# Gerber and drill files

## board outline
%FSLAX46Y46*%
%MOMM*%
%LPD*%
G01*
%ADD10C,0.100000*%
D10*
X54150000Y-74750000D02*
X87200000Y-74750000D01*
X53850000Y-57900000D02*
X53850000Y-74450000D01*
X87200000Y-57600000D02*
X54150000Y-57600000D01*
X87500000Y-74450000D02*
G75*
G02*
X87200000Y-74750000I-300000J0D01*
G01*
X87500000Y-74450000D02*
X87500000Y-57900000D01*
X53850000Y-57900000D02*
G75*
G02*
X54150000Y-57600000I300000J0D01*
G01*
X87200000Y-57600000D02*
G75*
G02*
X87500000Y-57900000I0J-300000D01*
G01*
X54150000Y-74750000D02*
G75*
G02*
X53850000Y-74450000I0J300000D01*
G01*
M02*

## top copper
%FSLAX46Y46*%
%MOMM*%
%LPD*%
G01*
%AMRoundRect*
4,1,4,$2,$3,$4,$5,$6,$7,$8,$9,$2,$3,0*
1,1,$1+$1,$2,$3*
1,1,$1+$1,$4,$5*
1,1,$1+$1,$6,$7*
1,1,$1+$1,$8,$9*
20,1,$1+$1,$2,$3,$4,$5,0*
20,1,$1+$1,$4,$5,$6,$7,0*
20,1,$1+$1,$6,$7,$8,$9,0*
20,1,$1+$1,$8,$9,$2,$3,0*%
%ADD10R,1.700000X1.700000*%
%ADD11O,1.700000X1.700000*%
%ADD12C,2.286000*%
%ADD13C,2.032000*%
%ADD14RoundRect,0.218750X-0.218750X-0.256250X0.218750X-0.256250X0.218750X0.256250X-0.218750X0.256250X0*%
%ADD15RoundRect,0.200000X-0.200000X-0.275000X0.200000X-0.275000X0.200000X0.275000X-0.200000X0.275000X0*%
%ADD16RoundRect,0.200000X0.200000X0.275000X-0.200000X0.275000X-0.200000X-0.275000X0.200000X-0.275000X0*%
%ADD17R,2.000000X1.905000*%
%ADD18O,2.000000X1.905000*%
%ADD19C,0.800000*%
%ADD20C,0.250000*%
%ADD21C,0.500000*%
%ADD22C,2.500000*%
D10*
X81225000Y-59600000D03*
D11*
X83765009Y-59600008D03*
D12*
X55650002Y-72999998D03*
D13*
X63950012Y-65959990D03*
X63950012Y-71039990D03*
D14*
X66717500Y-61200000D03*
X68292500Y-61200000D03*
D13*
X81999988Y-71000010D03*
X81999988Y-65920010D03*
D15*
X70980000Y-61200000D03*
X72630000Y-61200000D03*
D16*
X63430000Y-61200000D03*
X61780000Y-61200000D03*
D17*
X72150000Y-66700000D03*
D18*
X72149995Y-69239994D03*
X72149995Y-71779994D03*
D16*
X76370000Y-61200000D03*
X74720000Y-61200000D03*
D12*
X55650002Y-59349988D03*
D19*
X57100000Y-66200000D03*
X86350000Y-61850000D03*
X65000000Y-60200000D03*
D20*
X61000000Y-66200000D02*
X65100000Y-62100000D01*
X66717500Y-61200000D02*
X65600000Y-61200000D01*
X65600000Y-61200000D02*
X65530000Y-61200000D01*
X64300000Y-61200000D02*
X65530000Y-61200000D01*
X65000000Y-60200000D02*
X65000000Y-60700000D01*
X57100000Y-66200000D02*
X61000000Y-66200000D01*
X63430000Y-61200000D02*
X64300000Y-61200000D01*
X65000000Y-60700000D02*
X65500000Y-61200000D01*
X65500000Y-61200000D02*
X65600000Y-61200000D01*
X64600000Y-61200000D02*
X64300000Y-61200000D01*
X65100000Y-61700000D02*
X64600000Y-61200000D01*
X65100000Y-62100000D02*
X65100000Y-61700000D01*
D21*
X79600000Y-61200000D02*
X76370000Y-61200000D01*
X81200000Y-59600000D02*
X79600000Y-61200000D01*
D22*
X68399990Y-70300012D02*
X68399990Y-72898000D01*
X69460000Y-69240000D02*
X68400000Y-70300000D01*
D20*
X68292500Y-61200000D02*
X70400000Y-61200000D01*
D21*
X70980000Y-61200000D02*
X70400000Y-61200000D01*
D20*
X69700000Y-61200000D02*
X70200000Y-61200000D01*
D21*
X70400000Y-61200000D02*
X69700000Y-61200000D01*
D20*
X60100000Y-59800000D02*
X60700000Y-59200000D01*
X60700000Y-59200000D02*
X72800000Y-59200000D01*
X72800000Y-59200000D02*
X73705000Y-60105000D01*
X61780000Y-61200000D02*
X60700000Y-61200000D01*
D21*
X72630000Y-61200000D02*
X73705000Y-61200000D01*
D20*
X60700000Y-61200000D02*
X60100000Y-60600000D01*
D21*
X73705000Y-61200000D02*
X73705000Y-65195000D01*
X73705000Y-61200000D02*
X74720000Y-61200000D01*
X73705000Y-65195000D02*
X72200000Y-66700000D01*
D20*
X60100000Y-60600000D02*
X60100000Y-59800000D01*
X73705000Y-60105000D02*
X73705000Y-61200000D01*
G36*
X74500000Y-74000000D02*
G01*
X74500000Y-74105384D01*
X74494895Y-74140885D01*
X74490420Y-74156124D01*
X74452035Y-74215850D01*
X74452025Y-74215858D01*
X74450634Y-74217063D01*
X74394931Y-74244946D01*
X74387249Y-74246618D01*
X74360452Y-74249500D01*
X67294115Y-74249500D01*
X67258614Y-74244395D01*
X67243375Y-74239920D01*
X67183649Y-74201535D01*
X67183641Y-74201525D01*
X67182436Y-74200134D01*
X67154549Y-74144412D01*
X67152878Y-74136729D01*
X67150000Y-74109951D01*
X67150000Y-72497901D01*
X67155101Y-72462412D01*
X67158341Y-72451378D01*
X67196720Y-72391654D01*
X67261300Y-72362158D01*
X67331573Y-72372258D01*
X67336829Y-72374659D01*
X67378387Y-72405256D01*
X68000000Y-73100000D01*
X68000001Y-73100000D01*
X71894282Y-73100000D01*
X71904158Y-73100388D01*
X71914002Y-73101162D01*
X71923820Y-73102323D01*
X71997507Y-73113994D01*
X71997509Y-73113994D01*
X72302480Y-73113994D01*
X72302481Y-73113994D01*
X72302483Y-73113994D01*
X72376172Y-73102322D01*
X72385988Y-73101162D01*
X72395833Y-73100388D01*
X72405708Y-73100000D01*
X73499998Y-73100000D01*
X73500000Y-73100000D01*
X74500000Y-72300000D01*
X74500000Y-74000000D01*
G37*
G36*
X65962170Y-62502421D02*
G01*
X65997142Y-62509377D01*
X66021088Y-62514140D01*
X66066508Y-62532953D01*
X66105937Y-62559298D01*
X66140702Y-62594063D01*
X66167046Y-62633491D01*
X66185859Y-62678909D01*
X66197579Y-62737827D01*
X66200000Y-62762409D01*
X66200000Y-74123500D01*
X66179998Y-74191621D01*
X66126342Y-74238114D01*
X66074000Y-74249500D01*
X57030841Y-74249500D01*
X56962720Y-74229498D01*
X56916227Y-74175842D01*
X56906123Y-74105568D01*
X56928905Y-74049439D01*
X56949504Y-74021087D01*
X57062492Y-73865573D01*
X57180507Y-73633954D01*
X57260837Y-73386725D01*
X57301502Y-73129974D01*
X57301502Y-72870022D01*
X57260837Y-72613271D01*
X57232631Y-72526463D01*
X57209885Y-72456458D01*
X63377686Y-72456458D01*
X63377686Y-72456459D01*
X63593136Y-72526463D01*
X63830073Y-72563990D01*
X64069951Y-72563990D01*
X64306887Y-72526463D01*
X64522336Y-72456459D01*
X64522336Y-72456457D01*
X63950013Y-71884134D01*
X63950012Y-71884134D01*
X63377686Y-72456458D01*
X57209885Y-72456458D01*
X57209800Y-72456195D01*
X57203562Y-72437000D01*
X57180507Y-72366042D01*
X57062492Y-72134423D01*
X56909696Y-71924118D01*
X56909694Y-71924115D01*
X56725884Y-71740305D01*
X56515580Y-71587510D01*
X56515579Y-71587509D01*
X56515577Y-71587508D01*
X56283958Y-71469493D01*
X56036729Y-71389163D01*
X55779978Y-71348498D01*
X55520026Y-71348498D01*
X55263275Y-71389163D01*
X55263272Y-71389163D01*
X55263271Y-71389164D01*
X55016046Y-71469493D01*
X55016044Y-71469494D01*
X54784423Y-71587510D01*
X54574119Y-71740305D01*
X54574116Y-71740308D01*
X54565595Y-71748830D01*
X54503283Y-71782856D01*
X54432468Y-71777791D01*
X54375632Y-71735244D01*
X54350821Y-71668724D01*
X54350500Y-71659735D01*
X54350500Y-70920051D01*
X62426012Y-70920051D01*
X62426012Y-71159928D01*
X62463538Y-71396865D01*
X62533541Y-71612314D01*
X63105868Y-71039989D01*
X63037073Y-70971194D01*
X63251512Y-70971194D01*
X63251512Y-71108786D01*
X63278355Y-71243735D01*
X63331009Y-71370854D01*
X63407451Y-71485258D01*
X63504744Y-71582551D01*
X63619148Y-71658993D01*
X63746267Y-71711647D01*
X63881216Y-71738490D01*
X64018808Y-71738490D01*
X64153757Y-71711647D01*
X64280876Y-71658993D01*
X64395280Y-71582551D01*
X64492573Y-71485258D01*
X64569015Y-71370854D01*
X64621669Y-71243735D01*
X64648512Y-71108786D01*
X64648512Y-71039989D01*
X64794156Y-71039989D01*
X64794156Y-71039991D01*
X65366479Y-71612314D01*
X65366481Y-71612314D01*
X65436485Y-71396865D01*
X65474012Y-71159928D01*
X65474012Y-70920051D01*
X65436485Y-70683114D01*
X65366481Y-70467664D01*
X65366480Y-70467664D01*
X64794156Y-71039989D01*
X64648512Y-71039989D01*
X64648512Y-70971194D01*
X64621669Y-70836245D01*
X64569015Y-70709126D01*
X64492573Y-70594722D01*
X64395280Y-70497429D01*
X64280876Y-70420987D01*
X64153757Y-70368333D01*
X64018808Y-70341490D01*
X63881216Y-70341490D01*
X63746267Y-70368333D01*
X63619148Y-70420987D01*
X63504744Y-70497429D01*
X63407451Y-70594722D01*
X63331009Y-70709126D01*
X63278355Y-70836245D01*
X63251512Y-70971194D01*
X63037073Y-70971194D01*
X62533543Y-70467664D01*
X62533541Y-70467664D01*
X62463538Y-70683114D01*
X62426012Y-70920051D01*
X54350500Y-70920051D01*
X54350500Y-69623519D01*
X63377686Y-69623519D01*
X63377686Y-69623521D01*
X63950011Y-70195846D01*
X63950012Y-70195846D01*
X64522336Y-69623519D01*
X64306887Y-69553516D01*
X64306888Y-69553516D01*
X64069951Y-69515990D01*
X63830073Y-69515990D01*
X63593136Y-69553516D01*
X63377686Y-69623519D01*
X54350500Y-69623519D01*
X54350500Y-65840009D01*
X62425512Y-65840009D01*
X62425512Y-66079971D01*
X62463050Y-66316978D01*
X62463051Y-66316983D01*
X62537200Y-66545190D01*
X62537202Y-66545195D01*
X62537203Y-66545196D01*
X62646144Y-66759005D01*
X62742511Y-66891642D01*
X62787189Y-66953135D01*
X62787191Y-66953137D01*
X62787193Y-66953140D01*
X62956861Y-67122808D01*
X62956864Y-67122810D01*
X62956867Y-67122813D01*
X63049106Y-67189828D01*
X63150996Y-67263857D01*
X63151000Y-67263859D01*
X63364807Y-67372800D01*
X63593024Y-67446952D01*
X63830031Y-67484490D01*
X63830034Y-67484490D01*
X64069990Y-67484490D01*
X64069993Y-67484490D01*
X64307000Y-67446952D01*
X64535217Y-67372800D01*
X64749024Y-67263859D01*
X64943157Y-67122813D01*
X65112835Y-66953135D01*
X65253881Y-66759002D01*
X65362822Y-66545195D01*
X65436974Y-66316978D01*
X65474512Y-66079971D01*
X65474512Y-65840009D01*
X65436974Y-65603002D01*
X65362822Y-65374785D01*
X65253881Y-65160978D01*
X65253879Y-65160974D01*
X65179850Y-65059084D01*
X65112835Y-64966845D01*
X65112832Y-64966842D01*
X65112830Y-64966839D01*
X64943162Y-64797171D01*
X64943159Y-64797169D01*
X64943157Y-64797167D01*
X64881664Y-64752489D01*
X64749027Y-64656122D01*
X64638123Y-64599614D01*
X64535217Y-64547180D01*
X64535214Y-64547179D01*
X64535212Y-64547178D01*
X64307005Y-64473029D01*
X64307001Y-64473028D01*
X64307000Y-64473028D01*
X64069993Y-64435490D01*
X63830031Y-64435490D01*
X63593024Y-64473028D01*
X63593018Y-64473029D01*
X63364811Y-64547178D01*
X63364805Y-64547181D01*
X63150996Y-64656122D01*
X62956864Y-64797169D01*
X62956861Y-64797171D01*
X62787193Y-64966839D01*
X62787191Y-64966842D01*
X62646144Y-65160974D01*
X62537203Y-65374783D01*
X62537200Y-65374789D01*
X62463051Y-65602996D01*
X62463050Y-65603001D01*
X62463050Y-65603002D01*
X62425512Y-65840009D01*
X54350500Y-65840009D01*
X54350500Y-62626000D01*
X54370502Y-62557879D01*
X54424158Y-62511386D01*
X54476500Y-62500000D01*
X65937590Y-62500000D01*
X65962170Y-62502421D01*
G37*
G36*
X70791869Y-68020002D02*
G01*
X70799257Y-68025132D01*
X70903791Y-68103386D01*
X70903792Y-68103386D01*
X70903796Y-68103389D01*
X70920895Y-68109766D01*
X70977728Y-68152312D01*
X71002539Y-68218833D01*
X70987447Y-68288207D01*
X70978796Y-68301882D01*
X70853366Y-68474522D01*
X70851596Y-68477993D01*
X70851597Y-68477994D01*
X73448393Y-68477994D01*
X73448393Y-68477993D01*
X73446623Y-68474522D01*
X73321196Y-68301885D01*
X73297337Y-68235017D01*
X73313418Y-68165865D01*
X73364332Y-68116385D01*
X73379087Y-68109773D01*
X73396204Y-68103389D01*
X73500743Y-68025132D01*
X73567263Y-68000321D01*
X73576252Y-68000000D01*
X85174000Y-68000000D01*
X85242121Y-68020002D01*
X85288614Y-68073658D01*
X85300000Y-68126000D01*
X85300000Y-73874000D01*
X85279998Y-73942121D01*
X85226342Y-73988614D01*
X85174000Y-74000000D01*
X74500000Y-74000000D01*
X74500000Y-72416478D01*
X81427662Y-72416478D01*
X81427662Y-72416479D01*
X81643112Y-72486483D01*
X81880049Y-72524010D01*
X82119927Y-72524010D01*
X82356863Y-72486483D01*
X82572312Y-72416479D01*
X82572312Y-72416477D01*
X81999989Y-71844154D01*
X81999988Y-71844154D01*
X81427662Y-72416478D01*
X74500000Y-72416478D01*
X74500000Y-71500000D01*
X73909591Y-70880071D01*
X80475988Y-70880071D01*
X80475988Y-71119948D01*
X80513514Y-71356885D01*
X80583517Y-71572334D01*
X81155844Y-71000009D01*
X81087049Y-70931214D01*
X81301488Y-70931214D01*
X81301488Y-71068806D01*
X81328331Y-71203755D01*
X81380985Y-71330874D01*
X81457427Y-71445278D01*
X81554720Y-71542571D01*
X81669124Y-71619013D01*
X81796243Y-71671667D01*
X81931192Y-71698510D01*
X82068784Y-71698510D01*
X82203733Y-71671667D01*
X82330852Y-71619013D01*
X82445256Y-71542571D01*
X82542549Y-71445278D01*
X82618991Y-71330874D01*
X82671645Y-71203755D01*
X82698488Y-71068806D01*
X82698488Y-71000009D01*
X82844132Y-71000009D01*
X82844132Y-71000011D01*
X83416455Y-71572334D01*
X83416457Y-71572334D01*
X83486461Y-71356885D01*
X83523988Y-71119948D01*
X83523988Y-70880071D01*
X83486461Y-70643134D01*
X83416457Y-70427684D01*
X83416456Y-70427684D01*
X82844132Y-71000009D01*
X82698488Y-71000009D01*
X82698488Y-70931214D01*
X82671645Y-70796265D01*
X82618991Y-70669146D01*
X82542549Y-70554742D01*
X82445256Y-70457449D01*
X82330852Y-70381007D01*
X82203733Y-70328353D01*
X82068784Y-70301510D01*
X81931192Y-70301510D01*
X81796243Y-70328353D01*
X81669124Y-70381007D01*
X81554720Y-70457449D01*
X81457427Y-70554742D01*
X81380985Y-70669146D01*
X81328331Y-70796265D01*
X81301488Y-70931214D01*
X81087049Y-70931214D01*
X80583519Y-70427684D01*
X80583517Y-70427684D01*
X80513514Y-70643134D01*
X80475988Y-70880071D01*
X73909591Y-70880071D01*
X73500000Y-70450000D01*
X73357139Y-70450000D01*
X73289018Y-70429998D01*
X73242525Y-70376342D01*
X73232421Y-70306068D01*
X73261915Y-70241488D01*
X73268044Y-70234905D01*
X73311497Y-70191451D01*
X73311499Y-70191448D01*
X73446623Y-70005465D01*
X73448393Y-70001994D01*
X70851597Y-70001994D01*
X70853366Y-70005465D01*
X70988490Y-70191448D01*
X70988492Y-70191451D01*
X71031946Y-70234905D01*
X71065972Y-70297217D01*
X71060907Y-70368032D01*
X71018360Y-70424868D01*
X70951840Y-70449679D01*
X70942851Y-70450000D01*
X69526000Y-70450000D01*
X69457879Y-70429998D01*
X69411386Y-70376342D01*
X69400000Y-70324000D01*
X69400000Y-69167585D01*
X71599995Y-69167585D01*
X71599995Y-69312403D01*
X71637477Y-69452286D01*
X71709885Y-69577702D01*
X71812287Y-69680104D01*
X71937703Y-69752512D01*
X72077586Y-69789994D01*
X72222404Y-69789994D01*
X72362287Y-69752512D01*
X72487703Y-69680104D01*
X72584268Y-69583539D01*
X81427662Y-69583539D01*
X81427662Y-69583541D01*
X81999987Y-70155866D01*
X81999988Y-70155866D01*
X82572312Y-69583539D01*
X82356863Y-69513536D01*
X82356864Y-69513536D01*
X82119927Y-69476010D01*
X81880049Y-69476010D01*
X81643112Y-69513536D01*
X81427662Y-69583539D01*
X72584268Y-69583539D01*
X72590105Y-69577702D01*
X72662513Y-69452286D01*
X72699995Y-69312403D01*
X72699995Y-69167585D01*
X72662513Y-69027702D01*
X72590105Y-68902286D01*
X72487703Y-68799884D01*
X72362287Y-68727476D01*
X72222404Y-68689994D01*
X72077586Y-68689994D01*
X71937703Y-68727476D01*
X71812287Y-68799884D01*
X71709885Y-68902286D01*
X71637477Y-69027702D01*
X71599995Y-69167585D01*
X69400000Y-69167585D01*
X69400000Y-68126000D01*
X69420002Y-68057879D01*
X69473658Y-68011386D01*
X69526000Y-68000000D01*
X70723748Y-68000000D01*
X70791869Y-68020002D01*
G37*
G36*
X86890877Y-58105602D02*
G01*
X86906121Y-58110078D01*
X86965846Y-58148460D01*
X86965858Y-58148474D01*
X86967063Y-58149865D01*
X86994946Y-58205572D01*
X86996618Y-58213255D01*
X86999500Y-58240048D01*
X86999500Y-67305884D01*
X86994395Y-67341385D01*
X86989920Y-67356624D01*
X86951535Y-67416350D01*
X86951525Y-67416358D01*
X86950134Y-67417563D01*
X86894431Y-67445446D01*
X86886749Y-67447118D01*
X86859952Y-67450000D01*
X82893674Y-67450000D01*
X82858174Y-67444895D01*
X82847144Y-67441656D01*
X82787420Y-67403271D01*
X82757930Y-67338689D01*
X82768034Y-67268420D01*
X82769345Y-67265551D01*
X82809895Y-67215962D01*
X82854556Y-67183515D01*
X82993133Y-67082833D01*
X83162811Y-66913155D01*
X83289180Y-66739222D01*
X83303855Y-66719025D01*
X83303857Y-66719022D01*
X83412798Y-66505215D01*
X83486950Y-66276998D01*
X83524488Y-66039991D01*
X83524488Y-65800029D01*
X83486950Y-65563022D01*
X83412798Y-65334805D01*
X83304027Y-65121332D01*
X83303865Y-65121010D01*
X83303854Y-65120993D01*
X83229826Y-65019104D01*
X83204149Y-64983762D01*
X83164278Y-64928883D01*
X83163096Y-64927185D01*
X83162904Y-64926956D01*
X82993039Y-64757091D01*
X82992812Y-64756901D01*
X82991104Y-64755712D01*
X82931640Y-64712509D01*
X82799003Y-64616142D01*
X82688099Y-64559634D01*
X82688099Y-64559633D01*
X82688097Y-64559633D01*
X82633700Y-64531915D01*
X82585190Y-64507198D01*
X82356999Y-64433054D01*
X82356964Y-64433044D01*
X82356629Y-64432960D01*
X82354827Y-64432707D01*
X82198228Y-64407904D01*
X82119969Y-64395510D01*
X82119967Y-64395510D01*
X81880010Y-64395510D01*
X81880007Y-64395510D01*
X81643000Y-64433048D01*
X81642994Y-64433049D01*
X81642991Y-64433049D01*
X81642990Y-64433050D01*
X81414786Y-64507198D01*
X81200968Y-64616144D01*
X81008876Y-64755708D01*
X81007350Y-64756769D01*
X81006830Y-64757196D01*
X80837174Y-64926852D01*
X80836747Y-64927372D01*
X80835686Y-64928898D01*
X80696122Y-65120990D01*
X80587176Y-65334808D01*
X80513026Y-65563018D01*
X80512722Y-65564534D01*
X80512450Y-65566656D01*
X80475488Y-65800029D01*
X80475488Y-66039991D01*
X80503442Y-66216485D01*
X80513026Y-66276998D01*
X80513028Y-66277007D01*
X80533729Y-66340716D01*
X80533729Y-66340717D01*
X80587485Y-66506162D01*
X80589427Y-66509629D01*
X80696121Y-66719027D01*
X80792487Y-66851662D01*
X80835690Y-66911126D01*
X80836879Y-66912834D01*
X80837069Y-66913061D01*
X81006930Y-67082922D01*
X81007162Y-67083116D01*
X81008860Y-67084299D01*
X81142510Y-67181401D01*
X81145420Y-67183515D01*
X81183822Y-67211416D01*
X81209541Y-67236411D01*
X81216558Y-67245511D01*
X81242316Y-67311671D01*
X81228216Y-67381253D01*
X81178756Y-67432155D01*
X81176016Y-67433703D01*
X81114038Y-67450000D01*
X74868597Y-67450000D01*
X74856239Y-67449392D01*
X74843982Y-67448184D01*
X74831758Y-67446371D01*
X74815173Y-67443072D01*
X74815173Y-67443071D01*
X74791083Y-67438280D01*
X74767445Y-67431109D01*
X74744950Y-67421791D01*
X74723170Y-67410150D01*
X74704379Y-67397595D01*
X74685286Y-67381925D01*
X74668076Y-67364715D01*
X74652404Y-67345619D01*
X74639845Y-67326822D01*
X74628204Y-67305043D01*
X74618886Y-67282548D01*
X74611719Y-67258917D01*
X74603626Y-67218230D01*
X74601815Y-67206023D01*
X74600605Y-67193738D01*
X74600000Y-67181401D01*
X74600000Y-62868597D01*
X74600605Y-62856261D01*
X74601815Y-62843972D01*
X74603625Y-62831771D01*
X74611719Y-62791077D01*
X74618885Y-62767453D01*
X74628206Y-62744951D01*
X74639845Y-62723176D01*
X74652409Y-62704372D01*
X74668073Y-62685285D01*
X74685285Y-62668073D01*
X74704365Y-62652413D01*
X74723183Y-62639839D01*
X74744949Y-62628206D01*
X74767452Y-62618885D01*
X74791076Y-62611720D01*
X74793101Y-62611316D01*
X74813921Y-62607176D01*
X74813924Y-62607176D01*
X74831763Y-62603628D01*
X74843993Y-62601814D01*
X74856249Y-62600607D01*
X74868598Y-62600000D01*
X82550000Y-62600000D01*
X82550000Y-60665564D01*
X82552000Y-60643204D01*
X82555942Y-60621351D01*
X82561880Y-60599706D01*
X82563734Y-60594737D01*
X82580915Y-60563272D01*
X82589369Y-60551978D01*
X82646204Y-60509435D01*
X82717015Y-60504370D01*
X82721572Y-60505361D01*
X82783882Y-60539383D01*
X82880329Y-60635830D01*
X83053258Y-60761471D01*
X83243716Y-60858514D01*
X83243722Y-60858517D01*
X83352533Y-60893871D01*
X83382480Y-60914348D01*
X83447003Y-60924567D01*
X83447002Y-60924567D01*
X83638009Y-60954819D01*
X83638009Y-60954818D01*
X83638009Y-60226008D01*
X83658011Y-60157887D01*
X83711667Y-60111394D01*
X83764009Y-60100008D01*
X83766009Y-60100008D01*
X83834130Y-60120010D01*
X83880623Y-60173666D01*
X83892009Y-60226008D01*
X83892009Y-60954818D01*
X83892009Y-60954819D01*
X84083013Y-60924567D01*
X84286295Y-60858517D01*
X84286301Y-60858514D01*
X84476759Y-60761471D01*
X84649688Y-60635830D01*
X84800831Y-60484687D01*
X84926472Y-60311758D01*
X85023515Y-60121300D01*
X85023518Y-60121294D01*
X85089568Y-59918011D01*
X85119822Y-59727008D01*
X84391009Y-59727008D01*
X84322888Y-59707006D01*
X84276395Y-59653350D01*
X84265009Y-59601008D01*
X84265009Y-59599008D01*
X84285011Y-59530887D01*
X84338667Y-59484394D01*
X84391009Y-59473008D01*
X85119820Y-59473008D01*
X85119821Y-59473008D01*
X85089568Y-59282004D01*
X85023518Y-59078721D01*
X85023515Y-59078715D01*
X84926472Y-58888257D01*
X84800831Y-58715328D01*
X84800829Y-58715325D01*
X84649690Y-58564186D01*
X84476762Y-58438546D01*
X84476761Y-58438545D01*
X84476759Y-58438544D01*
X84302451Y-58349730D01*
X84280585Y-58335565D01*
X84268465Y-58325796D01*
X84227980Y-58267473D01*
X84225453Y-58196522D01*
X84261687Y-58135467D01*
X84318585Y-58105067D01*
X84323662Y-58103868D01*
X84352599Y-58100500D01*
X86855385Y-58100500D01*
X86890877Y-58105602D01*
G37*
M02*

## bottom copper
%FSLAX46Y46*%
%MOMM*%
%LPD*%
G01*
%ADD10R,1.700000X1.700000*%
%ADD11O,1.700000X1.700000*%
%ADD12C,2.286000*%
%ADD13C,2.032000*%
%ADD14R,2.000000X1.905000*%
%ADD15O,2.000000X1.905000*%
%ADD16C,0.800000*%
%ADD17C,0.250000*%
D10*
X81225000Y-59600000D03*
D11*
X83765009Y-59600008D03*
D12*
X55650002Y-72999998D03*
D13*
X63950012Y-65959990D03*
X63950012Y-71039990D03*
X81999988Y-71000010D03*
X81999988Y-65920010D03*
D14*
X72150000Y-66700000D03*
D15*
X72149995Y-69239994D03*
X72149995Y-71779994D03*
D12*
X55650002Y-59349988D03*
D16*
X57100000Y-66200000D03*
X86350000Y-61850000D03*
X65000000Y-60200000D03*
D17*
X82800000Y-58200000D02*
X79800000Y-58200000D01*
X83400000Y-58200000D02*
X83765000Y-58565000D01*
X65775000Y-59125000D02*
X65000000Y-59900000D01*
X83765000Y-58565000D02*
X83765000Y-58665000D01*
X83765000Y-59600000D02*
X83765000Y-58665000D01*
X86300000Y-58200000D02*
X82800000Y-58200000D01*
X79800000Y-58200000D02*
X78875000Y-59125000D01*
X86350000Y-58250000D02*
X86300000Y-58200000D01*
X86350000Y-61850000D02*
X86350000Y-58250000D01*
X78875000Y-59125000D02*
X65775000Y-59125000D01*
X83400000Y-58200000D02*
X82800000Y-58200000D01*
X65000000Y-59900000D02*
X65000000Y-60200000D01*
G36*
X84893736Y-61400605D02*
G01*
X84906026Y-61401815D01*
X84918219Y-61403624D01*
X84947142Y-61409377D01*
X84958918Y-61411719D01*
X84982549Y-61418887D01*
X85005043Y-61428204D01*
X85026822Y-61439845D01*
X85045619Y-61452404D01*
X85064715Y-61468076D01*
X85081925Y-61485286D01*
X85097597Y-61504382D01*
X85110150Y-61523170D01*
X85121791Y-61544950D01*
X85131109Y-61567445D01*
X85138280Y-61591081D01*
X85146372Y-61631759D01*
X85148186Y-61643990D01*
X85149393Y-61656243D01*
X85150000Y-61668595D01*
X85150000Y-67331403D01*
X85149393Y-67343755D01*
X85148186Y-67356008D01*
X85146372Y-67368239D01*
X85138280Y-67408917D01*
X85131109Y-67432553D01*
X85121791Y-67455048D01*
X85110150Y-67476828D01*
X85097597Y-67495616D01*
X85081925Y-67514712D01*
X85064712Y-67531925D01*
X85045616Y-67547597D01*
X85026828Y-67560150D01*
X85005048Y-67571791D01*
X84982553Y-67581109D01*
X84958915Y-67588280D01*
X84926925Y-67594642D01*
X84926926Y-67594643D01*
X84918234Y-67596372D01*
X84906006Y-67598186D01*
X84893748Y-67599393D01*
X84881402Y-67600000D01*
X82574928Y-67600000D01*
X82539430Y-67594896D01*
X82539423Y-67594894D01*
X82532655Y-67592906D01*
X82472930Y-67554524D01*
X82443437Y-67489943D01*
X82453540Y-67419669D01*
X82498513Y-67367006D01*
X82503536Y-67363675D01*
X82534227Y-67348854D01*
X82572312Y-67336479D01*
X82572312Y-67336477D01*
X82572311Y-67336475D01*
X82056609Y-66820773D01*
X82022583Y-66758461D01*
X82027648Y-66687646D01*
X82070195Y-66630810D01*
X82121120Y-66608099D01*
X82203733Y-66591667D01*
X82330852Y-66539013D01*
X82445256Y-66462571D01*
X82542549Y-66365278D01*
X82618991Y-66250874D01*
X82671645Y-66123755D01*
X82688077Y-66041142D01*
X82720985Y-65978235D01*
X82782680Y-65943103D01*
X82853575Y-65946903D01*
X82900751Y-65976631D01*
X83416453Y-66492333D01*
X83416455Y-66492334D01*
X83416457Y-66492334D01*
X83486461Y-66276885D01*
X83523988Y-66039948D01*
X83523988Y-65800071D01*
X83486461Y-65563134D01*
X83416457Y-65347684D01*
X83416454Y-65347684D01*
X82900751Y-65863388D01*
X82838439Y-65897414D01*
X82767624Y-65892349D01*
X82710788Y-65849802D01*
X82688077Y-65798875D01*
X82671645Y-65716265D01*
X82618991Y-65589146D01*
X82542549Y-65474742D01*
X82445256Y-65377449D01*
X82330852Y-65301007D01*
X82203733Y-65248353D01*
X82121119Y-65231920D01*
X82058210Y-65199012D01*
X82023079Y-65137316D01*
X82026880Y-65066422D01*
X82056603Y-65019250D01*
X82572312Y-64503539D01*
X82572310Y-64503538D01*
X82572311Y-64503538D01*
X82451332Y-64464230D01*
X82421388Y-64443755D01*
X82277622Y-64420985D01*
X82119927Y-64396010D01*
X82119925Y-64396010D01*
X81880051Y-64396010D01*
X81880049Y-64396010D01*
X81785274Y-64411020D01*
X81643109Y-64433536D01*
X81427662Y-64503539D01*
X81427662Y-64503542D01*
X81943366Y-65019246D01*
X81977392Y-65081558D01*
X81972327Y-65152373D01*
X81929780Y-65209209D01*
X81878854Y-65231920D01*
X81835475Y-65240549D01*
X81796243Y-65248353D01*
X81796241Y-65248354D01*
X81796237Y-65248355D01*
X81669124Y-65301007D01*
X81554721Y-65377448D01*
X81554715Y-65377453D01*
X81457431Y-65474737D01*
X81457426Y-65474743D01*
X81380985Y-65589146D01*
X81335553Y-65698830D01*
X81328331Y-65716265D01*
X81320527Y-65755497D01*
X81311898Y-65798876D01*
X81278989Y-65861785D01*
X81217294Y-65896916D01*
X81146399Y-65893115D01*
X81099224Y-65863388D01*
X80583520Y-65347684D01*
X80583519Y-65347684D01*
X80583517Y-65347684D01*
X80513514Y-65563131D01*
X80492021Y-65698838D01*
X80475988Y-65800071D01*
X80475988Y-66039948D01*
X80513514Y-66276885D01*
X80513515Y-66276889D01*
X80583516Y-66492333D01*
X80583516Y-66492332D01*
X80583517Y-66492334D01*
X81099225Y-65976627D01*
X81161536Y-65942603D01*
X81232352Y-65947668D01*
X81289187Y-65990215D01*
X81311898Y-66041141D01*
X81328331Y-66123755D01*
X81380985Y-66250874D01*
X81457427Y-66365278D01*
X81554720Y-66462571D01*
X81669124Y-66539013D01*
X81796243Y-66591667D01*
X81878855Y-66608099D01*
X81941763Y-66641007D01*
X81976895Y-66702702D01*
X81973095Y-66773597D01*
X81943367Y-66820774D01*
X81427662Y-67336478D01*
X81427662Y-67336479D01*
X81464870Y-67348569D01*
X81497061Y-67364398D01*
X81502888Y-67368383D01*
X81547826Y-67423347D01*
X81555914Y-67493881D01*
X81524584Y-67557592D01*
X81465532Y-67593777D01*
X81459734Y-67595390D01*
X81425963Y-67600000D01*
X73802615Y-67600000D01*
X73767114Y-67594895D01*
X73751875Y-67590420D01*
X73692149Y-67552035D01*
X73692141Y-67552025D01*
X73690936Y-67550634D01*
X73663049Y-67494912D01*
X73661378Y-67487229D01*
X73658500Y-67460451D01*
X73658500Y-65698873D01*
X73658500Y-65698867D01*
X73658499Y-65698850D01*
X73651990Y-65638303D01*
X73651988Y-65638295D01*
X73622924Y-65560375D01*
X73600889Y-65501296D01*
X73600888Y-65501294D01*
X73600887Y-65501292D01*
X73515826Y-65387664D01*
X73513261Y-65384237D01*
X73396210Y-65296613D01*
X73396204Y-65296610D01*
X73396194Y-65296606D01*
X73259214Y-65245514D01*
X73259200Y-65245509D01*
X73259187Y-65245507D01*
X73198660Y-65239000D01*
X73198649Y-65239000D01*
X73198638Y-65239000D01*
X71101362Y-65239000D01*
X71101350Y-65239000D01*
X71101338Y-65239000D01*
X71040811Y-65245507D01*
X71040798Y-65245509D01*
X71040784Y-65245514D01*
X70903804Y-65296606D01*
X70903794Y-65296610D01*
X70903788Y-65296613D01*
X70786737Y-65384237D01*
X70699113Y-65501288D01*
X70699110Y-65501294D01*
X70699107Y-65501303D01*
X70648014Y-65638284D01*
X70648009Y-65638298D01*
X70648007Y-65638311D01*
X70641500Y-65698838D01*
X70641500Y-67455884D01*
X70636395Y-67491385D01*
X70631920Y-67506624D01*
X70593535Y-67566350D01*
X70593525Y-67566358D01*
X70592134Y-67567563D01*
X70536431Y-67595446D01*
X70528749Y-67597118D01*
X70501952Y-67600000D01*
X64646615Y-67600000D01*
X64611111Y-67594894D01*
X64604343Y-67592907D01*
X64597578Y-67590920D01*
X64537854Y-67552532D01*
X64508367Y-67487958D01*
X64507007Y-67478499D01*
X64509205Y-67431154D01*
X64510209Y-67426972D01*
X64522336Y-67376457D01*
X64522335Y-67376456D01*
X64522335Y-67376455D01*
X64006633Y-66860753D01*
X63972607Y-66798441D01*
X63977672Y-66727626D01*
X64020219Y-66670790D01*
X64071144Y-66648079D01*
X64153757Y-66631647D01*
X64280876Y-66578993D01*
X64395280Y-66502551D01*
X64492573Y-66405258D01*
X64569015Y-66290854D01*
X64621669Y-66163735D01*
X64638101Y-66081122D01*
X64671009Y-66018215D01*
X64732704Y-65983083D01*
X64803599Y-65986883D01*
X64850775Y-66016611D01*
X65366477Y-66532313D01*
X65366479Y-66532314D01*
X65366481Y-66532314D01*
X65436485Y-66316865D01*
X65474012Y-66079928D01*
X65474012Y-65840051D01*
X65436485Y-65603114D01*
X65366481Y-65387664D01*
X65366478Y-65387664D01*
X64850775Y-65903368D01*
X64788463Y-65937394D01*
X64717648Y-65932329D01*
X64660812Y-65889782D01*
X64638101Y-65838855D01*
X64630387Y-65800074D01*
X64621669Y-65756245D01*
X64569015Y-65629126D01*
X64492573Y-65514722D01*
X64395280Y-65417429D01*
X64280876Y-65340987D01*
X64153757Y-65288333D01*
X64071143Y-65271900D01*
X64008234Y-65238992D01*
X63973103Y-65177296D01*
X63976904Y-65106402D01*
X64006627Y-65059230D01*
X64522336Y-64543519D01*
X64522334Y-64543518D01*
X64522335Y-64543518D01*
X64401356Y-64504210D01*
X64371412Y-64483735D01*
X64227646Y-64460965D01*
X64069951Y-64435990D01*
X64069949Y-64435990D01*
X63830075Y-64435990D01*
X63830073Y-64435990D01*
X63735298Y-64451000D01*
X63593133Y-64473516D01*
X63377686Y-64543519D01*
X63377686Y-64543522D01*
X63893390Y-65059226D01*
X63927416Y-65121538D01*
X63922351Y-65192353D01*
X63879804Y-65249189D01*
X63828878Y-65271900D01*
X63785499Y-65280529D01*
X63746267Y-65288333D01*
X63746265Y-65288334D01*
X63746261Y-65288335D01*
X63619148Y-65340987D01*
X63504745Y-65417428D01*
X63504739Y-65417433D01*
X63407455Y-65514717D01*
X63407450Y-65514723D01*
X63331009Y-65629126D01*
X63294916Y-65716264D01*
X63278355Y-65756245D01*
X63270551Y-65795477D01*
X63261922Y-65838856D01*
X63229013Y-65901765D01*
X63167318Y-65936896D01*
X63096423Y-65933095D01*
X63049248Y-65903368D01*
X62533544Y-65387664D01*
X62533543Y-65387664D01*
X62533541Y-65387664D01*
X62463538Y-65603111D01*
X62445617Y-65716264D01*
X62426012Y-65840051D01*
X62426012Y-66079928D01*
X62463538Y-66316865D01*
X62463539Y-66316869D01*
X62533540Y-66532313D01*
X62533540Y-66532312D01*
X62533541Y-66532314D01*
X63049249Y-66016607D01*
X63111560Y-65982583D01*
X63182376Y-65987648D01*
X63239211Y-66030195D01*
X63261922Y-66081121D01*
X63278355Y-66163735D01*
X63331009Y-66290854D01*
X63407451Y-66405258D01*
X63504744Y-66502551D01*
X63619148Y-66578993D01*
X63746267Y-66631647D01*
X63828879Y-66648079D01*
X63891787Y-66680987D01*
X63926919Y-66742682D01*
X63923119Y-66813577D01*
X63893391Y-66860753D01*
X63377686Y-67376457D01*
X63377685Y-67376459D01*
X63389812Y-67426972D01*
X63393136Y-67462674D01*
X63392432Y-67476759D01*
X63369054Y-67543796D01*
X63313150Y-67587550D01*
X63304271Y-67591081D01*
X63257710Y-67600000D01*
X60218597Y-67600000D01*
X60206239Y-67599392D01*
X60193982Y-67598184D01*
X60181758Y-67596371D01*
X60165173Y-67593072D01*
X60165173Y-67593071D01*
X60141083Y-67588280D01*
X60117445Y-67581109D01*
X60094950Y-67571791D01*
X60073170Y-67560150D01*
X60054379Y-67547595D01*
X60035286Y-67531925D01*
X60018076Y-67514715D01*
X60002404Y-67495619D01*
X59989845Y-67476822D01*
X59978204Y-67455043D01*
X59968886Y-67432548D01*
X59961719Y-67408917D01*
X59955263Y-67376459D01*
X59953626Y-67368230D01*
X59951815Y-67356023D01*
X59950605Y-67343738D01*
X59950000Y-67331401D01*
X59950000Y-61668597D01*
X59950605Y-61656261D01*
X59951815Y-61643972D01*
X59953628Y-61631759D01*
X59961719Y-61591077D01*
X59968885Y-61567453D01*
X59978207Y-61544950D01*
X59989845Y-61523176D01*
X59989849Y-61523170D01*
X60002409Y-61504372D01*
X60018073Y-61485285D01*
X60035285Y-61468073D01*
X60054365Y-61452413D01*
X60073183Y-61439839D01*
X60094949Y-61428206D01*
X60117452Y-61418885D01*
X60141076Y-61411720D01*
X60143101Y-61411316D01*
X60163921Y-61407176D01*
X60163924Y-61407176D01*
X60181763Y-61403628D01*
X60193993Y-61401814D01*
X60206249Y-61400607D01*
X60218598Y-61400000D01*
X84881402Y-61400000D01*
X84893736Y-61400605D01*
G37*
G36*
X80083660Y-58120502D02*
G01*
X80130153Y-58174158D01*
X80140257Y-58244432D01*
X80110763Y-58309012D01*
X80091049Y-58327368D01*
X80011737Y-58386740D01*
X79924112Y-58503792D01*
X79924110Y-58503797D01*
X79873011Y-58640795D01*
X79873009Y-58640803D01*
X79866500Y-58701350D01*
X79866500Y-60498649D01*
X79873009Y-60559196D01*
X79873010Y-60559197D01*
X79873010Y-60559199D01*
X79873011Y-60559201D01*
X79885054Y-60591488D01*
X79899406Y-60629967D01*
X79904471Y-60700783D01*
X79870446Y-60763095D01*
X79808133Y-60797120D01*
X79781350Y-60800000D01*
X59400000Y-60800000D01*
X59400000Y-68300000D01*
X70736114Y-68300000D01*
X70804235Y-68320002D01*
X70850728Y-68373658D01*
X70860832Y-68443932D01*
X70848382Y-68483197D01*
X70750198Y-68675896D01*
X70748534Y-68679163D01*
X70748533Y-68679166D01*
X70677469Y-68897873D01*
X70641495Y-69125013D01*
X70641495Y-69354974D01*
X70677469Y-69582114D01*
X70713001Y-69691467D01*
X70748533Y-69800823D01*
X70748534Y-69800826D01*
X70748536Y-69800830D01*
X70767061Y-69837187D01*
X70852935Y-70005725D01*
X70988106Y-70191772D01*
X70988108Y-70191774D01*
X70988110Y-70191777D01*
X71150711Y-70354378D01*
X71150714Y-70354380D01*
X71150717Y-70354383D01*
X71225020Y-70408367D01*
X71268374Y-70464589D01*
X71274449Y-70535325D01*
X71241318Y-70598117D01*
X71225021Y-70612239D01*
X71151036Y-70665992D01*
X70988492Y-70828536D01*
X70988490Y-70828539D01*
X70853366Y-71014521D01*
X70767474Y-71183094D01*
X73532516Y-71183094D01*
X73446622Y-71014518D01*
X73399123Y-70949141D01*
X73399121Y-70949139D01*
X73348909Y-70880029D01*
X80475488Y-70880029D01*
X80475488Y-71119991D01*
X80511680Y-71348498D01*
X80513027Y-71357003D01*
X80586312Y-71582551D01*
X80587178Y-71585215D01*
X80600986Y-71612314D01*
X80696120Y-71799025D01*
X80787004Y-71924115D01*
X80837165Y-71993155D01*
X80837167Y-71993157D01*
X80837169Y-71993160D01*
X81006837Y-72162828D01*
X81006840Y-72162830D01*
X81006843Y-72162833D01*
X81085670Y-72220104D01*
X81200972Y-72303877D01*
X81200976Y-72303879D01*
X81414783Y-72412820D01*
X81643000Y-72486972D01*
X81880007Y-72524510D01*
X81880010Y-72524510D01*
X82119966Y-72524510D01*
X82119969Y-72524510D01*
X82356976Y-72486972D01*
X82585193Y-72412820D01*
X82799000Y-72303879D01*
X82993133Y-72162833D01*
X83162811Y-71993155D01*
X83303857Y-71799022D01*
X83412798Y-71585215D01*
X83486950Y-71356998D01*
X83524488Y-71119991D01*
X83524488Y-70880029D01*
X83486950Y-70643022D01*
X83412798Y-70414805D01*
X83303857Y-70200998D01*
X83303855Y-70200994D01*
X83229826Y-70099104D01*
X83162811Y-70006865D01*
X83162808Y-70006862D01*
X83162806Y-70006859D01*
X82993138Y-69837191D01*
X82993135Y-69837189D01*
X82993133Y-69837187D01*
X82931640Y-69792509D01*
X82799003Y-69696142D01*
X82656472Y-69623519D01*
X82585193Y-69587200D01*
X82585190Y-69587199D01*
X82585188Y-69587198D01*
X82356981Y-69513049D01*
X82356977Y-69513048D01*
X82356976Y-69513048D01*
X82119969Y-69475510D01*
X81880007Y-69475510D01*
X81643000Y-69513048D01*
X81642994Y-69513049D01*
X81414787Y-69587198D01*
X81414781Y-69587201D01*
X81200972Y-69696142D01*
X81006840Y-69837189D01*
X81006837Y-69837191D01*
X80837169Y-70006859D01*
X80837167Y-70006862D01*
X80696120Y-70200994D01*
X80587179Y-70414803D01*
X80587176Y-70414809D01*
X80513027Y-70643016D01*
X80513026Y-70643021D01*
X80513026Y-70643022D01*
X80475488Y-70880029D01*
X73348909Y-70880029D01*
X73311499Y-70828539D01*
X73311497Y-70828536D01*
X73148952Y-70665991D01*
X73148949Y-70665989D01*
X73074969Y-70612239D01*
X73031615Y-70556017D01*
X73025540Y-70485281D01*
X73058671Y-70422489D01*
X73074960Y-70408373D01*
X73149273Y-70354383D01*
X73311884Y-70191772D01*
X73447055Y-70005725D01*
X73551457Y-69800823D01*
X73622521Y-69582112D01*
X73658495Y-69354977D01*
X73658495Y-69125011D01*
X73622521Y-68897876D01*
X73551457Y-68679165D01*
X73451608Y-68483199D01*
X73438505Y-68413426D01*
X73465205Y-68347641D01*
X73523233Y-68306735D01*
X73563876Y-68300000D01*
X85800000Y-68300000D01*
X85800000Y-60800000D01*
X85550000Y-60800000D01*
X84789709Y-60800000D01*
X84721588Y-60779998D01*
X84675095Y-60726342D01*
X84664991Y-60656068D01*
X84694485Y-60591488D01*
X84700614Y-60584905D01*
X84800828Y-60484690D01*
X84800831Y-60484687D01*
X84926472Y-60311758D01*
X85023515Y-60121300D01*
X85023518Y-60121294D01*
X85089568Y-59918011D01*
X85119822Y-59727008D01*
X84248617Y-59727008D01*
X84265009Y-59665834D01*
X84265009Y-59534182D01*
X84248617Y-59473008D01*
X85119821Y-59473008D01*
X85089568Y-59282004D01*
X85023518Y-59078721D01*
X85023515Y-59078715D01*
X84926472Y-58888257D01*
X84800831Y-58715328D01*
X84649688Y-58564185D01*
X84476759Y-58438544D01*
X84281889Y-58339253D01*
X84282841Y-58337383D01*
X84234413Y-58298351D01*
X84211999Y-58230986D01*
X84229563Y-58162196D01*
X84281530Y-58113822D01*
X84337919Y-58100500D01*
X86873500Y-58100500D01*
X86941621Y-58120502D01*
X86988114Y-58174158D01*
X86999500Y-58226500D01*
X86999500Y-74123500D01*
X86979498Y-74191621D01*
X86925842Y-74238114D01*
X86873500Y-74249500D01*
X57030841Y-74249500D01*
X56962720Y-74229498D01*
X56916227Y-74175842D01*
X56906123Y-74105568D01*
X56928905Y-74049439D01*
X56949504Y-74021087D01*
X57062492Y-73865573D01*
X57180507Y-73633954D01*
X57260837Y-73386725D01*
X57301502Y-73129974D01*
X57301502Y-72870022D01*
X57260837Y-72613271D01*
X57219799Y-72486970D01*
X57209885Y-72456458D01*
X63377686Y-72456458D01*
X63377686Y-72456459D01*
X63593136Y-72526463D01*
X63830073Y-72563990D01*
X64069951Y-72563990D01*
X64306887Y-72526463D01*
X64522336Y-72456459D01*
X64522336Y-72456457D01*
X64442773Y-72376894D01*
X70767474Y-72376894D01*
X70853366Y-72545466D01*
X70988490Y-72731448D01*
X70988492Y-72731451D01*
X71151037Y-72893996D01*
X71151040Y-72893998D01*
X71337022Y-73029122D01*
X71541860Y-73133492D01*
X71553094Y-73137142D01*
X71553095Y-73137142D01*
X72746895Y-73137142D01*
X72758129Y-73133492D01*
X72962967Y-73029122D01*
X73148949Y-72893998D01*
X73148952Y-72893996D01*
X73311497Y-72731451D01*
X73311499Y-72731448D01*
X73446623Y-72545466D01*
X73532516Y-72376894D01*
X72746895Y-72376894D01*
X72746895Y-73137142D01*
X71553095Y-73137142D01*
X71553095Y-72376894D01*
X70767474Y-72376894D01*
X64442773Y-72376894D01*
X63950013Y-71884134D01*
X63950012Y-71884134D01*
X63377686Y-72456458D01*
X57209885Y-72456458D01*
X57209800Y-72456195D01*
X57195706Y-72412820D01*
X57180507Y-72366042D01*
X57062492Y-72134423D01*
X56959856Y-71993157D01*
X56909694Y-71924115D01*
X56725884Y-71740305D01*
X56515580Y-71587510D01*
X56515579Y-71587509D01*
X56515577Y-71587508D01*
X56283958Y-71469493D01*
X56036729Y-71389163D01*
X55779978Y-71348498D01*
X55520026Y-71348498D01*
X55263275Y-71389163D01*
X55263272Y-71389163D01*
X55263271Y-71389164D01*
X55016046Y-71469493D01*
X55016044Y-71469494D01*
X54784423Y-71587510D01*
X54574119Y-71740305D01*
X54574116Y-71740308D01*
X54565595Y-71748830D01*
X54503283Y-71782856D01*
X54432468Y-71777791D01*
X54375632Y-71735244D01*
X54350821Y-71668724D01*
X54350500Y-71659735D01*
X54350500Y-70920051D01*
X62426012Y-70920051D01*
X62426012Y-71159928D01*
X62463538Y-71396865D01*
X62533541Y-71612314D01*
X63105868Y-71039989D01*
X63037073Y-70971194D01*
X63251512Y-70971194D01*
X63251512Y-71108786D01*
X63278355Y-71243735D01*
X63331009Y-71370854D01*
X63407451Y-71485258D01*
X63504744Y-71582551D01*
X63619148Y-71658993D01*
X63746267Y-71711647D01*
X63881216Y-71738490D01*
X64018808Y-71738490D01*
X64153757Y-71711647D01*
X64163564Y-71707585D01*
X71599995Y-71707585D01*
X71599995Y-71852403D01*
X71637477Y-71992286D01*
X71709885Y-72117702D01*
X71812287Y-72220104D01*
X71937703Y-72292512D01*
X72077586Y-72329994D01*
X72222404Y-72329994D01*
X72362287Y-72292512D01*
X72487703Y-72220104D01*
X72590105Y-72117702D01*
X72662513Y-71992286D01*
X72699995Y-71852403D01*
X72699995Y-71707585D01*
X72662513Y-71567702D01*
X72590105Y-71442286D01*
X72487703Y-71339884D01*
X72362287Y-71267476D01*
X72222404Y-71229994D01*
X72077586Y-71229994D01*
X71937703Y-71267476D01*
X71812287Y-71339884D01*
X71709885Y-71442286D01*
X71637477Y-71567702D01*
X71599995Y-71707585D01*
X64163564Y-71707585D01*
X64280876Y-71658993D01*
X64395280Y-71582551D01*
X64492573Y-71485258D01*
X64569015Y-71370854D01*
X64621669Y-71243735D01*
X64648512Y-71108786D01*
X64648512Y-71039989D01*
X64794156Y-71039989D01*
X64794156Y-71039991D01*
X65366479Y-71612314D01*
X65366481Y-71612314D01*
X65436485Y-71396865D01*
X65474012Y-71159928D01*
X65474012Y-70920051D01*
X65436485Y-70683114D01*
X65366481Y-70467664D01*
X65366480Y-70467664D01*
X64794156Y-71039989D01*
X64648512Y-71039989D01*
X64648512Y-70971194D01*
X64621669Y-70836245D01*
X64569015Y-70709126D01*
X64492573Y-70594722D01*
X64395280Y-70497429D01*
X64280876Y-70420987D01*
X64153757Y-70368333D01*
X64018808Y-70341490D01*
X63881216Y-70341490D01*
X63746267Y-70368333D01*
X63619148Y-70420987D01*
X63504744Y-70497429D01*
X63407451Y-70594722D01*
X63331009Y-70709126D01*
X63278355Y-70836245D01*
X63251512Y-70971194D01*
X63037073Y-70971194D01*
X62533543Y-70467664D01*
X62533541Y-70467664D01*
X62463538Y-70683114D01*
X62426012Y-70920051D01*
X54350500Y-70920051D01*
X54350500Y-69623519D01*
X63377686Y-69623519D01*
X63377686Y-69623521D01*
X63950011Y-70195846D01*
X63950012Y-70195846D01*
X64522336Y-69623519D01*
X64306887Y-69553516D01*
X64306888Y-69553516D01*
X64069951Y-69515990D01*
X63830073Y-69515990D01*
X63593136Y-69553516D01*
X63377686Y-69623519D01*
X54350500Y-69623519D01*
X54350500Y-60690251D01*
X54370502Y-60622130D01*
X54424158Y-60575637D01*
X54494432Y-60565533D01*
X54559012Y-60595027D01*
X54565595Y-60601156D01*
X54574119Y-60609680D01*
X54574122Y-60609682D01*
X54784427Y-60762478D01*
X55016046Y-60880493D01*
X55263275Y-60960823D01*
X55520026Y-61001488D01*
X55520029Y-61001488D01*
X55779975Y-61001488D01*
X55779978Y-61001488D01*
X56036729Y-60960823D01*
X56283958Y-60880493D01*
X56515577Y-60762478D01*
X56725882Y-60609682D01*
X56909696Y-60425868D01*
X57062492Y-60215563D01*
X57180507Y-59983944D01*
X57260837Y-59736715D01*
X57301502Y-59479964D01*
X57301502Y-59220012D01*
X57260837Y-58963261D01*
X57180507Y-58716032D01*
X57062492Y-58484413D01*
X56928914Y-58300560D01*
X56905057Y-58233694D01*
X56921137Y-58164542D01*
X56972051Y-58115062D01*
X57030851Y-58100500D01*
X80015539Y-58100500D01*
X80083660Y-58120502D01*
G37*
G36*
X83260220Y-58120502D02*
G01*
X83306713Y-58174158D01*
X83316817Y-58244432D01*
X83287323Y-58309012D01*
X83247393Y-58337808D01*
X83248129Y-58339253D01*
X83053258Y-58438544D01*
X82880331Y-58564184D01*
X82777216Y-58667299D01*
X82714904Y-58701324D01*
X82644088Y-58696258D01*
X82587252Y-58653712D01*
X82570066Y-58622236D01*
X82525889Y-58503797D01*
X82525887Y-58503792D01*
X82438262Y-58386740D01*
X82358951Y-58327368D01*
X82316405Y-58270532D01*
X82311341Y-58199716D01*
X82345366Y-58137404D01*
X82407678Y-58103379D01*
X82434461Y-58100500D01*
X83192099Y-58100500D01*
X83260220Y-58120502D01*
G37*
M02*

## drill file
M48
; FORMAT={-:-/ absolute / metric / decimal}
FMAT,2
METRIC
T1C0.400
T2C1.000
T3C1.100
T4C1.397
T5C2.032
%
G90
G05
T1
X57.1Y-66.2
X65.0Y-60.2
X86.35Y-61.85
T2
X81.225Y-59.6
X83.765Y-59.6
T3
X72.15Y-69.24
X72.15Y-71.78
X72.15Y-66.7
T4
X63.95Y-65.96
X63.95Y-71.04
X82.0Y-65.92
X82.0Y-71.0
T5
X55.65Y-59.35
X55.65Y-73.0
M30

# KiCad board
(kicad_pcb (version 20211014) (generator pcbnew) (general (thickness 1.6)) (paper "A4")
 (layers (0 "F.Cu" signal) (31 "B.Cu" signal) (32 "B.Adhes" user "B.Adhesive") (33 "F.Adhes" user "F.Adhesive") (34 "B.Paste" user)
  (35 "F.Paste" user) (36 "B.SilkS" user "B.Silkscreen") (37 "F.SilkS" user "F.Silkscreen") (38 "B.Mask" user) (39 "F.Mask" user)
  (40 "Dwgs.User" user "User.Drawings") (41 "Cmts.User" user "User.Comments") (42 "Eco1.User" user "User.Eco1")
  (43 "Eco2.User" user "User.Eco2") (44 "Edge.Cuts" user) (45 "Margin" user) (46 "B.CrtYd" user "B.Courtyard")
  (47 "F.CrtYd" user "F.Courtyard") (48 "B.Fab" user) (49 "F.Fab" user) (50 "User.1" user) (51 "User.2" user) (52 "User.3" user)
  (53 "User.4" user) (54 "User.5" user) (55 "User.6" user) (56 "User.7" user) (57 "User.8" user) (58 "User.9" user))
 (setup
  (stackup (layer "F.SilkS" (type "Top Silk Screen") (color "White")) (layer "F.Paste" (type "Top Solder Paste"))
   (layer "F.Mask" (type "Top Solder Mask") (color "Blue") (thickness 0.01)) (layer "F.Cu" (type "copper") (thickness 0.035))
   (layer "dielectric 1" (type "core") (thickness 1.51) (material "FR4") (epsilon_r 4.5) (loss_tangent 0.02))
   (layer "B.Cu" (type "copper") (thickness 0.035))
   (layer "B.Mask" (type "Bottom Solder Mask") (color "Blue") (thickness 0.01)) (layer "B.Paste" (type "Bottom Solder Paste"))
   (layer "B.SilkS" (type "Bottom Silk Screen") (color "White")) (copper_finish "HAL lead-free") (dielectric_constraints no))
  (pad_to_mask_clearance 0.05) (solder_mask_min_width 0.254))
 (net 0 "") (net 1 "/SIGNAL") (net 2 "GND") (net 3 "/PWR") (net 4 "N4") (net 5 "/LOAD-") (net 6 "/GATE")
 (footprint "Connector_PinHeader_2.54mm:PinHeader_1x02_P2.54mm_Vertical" (layer "F.Cu") (at 81.225 59.6 90)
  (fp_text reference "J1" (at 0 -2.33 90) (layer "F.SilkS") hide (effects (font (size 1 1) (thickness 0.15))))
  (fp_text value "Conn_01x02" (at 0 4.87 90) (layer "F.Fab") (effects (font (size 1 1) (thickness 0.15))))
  (pad "1" thru_hole rect (at 0 0 90) (size 1.7 1.7) (drill 1) (layers *.Cu *.Mask) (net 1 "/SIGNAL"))
  (pad "2" thru_hole oval (at -0.000008 2.540009 90) (size 1.7 1.7) (drill 1) (layers *.Cu *.Mask) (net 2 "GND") (thermal_width 0.254)))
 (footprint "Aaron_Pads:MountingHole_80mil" (layer "F.Cu") (at 55.650002 72.999998)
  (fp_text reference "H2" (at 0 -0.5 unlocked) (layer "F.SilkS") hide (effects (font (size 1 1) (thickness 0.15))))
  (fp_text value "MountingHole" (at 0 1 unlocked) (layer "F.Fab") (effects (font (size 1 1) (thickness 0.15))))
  (pad "" thru_hole circle (at 0 0) (size 2.286 2.286) (drill 2.032) (layers *.Cu *.Mask) (zone_connect 0)))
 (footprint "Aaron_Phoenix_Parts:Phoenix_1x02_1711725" (layer "F.Cu") (at 63.95 65.96 -90)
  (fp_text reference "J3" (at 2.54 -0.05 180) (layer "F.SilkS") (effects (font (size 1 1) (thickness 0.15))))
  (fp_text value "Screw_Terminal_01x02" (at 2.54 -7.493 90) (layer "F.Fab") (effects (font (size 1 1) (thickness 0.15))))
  (pad "1" thru_hole circle (at -0.00001 -0.000012 270) (size 2.032 2.032) (drill 1.397) (layers *.Cu *.Mask) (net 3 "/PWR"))
  (pad "2" thru_hole circle (at 5.07999 -0.000012 270) (size 2.032 2.032) (drill 1.397) (layers *.Cu *.Mask) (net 2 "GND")))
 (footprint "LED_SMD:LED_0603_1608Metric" (layer "F.Cu") (at 67.505 61.2)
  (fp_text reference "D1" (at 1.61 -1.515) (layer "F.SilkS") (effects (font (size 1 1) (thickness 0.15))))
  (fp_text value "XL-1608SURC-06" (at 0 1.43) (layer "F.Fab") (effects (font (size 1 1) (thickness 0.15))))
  (pad "1" smd roundrect (at -0.7875 0) (size 0.875 0.95) (layers "F.Cu" "F.Paste" "F.Mask") (roundrect_rratio 0.25) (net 2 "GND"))
  (pad "2" smd roundrect (at 0.7875 0) (size 0.875 0.95) (layers "F.Cu" "F.Paste" "F.Mask") (roundrect_rratio 0.25) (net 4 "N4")))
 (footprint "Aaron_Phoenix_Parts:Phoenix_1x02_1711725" (layer "F.Cu") (at 82 71 90)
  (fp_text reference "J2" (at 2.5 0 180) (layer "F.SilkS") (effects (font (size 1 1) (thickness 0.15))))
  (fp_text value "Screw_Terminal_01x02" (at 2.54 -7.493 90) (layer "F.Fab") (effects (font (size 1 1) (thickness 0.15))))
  (pad "1" thru_hole circle (at -0.00001 -0.000012 90) (size 2.032 2.032) (drill 1.397) (layers *.Cu *.Mask) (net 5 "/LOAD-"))
  (pad "2" thru_hole circle (at 5.07999 -0.000012 90) (size 2.032 2.032) (drill 1.397) (layers *.Cu *.Mask) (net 3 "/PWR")))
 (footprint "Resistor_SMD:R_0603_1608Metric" (layer "F.Cu") (at 71.805 61.2)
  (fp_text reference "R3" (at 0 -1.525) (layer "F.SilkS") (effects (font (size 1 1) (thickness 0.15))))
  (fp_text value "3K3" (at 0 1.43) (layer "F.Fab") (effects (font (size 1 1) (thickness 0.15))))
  (pad "1" smd roundrect (at -0.825 0) (size 0.8 0.95) (layers "F.Cu" "F.Paste" "F.Mask") (roundrect_rratio 0.25) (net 4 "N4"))
  (pad "2" smd roundrect (at 0.825 0) (size 0.8 0.95) (layers "F.Cu" "F.Paste" "F.Mask") (roundrect_rratio 0.25) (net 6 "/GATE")))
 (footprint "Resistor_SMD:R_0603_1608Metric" (layer "F.Cu") (at 62.605 61.2 180)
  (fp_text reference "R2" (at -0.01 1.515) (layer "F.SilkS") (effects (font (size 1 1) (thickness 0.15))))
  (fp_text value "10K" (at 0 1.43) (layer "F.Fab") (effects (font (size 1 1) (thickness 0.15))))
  (pad "1" smd roundrect (at -0.825 0 180) (size 0.8 0.95) (layers "F.Cu" "F.Paste" "F.Mask") (roundrect_rratio 0.25) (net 2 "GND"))
  (pad "2" smd roundrect (at 0.825 0 180) (size 0.8 0.95) (layers "F.Cu" "F.Paste" "F.Mask") (roundrect_rratio 0.25) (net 6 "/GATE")))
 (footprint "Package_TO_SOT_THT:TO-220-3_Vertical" (layer "F.Cu") (at 72.15 66.7 -90)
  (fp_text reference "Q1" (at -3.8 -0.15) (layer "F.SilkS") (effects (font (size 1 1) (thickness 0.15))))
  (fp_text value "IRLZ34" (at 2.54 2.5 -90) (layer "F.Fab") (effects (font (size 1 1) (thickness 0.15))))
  (pad "1" thru_hole rect (at 0 0 270) (size 1.905 2) (drill 1.1) (layers *.Cu *.Mask) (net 6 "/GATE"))
  (pad "2" thru_hole oval (at 2.539994 0.000005 270) (size 1.905 2) (drill 1.1) (layers *.Cu *.Mask) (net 5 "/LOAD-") (zone_connect 1)
   (thermal_width 1.524))
  (pad "3" thru_hole oval (at 5.079994 0.000005 270) (size 1.905 2) (drill 1.1) (layers *.Cu *.Mask) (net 2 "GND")))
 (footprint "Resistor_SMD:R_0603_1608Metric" (layer "F.Cu") (at 75.545 61.2 180)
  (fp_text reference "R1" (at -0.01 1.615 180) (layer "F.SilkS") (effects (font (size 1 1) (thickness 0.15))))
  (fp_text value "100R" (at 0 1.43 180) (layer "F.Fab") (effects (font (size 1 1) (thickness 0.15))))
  (pad "1" smd roundrect (at -0.825 0 180) (size 0.8 0.95) (layers "F.Cu" "F.Paste" "F.Mask") (roundrect_rratio 0.25) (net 1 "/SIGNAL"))
  (pad "2" smd roundrect (at 0.825 0 180) (size 0.8 0.95) (layers "F.Cu" "F.Paste" "F.Mask") (roundrect_rratio 0.25) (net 6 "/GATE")))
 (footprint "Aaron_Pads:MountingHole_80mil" (layer "F.Cu") (at 55.650002 59.349988)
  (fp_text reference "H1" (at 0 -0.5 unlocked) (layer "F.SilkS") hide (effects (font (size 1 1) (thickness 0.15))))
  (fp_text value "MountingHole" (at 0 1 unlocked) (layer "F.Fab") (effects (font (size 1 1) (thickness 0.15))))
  (pad "" thru_hole circle (at 0 0) (size 2.286 2.286) (drill 2.032) (layers *.Cu *.Mask) (zone_connect 0)))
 (gr_line (start 54.15 74.75) (end 87.2 74.75) (layer "Edge.Cuts") (width 0.1))
 (gr_line (start 53.85 57.9) (end 53.85 74.45) (layer "Edge.Cuts") (width 0.1))
 (gr_line (start 87.2 57.6) (end 54.15 57.6) (layer "Edge.Cuts") (width 0.1))
 (gr_arc (start 87.5 74.45) (mid 87.412132 74.662132) (end 87.2 74.75) (layer "Edge.Cuts") (width 0.1))
 (gr_line (start 87.5 74.45) (end 87.5 57.9) (layer "Edge.Cuts") (width 0.1))
 (gr_arc (start 53.85 57.9) (mid 53.937868 57.687868) (end 54.15 57.6) (layer "Edge.Cuts") (width 0.1))
 (gr_arc (start 87.2 57.6) (mid 87.412132 57.687868) (end 87.5 57.9) (layer "Edge.Cuts") (width 0.1))
 (gr_arc (start 54.15 74.75) (mid 53.937868 74.662132) (end 53.85 74.45) (layer "Edge.Cuts") (width 0.1))
 (segment (start 61 66.2) (end 65.1 62.1) (width 0.25) (layer "F.Cu") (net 2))
 (segment (start 66.7175 61.2) (end 65.6 61.2) (width 0.25) (layer "F.Cu") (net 2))
 (segment (start 65.6 61.2) (end 65.53 61.2) (width 0.25) (layer "F.Cu") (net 2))
 (segment (start 64.3 61.2) (end 65.53 61.2) (width 0.25) (layer "F.Cu") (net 2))
 (segment (start 65 60.2) (end 65 60.7) (width 0.25) (layer "F.Cu") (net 2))
 (segment (start 57.1 66.2) (end 61 66.2) (width 0.25) (layer "F.Cu") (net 2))
 (segment (start 63.43 61.2) (end 64.3 61.2) (width 0.25) (layer "F.Cu") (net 2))
 (segment (start 65 60.7) (end 65.5 61.2) (width 0.25) (layer "F.Cu") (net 2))
 (segment (start 65.5 61.2) (end 65.6 61.2) (width 0.25) (layer "F.Cu") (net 2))
 (segment (start 64.6 61.2) (end 64.3 61.2) (width 0.25) (layer "F.Cu") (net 2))
 (segment (start 65.1 61.7) (end 64.6 61.2) (width 0.25) (layer "F.Cu") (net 2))
 (segment (start 65.1 62.1) (end 65.1 61.7) (width 0.25) (layer "F.Cu") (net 2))
 (via (at 57.1 66.2) (size 0.8) (drill 0.4) (layers "F.Cu" "B.Cu") (free) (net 2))
 (via (at 86.35 61.85) (size 0.8) (drill 0.4) (layers "F.Cu" "B.Cu") (free) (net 2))
 (via (at 65 60.2) (size 0.8) (drill 0.4) (layers "F.Cu" "B.Cu") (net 2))
 (segment (start 82.8 58.2) (end 79.8 58.2) (width 0.25) (layer "B.Cu") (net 2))
 (segment (start 83.4 58.2) (end 83.765 58.565) (width 0.25) (layer "B.Cu") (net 2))
 (segment (start 65.775 59.125) (end 65 59.9) (width 0.25) (layer "B.Cu") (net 2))
 (segment (start 83.765 58.565) (end 83.765 58.665) (width 0.25) (layer "B.Cu") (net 2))
 (segment (start 83.765 59.6) (end 83.765 58.665) (width 0.25) (layer "B.Cu") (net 2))
 (segment (start 86.3 58.2) (end 82.8 58.2) (width 0.25) (layer "B.Cu") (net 2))
 (segment (start 79.8 58.2) (end 78.875 59.125) (width 0.25) (layer "B.Cu") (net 2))
 (segment (start 86.35 58.25) (end 86.3 58.2) (width 0.25) (layer "B.Cu") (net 2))
 (segment (start 86.35 61.85) (end 86.35 58.25) (width 0.25) (layer "B.Cu") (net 2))
 (segment (start 78.875 59.125) (end 65.775 59.125) (width 0.25) (layer "B.Cu") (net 2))
 (segment (start 83.4 58.2) (end 82.8 58.2) (width 0.25) (layer "B.Cu") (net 2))
 (segment (start 65 59.9) (end 65 60.2) (width 0.25) (layer "B.Cu") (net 2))
 (segment (start 79.6 61.2) (end 76.37 61.2) (width 0.5) (layer "F.Cu") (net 1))
 (segment (start 81.2 59.6) (end 79.6 61.2) (width 0.5) (layer "F.Cu") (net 1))
 (segment (start 68.39999 70.300012) (end 68.39999 72.898) (width 2.5) (layer "F.Cu") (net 5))
 (segment (start 69.46 69.24) (end 68.4 70.3) (width 2.5) (layer "F.Cu") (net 5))
 (segment (start 68.2925 61.2) (end 70.4 61.2) (width 0.25) (layer "F.Cu") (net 4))
 (segment (start 70.98 61.2) (end 70.4 61.2) (width 0.5) (layer "F.Cu") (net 4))
 (segment (start 69.7 61.2) (end 70.2 61.2) (width 0.25) (layer "F.Cu") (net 4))
 (segment (start 70.4 61.2) (end 69.7 61.2) (width 0.5) (layer "F.Cu") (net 4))
 (segment (start 60.1 59.8) (end 60.7 59.2) (width 0.25) (layer "F.Cu") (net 6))
 (segment (start 60.7 59.2) (end 72.8 59.2) (width 0.25) (layer "F.Cu") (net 6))
 (segment (start 72.8 59.2) (end 73.705 60.105) (width 0.25) (layer "F.Cu") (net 6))
 (segment (start 61.78 61.2) (end 60.7 61.2) (width 0.25) (layer "F.Cu") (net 6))
 (segment (start 72.63 61.2) (end 73.705 61.2) (width 0.5) (layer "F.Cu") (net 6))
 (segment (start 60.7 61.2) (end 60.1 60.6) (width 0.25) (layer "F.Cu") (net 6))
 (segment (start 73.705 61.2) (end 73.705 65.195) (width 0.5) (layer "F.Cu") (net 6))
 (segment (start 73.705 61.2) (end 74.72 61.2) (width 0.5) (layer "F.Cu") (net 6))
 (segment (start 73.705 65.195) (end 72.2 66.7) (width 0.5) (layer "F.Cu") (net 6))
 (segment (start 60.1 60.6) (end 60.1 59.8) (width 0.25) (layer "F.Cu") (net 6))
 (segment (start 73.705 60.105) (end 73.705 61.2) (width 0.25) (layer "F.Cu") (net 6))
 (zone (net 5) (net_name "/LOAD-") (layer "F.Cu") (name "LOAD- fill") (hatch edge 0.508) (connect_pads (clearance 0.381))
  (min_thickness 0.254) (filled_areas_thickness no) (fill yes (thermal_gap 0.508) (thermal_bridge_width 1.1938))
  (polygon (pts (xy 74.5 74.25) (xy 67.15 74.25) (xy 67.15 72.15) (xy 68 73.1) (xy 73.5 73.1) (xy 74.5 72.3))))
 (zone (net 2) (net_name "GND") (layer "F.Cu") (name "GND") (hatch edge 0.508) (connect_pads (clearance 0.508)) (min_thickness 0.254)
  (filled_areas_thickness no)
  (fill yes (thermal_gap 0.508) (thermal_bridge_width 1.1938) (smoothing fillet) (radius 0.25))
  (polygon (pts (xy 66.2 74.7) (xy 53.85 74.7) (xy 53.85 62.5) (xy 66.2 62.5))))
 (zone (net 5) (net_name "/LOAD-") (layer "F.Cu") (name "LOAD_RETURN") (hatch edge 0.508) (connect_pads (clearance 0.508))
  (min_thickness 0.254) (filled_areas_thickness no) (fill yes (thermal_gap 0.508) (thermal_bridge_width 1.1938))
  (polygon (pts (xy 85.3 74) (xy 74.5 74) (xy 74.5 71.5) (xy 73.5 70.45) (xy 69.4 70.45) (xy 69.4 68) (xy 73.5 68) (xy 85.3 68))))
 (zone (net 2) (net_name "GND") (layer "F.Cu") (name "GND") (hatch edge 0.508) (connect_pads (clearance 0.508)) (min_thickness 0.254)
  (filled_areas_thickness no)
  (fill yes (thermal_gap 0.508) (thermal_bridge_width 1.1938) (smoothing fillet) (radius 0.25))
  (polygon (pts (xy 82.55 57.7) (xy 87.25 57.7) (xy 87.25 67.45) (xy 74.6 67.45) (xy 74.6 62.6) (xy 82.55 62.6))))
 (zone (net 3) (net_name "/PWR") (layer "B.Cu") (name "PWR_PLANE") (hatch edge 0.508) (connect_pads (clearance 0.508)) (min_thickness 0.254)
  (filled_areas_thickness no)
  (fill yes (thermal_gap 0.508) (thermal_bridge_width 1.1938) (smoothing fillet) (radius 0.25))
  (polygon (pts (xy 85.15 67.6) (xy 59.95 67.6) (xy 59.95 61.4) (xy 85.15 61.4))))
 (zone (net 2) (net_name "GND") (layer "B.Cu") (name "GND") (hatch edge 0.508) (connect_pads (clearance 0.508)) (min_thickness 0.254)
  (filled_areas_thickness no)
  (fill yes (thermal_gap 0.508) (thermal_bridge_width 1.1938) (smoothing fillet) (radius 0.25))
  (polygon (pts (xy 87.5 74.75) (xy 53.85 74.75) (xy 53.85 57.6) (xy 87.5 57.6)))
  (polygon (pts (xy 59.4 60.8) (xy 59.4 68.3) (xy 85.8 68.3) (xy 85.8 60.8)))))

